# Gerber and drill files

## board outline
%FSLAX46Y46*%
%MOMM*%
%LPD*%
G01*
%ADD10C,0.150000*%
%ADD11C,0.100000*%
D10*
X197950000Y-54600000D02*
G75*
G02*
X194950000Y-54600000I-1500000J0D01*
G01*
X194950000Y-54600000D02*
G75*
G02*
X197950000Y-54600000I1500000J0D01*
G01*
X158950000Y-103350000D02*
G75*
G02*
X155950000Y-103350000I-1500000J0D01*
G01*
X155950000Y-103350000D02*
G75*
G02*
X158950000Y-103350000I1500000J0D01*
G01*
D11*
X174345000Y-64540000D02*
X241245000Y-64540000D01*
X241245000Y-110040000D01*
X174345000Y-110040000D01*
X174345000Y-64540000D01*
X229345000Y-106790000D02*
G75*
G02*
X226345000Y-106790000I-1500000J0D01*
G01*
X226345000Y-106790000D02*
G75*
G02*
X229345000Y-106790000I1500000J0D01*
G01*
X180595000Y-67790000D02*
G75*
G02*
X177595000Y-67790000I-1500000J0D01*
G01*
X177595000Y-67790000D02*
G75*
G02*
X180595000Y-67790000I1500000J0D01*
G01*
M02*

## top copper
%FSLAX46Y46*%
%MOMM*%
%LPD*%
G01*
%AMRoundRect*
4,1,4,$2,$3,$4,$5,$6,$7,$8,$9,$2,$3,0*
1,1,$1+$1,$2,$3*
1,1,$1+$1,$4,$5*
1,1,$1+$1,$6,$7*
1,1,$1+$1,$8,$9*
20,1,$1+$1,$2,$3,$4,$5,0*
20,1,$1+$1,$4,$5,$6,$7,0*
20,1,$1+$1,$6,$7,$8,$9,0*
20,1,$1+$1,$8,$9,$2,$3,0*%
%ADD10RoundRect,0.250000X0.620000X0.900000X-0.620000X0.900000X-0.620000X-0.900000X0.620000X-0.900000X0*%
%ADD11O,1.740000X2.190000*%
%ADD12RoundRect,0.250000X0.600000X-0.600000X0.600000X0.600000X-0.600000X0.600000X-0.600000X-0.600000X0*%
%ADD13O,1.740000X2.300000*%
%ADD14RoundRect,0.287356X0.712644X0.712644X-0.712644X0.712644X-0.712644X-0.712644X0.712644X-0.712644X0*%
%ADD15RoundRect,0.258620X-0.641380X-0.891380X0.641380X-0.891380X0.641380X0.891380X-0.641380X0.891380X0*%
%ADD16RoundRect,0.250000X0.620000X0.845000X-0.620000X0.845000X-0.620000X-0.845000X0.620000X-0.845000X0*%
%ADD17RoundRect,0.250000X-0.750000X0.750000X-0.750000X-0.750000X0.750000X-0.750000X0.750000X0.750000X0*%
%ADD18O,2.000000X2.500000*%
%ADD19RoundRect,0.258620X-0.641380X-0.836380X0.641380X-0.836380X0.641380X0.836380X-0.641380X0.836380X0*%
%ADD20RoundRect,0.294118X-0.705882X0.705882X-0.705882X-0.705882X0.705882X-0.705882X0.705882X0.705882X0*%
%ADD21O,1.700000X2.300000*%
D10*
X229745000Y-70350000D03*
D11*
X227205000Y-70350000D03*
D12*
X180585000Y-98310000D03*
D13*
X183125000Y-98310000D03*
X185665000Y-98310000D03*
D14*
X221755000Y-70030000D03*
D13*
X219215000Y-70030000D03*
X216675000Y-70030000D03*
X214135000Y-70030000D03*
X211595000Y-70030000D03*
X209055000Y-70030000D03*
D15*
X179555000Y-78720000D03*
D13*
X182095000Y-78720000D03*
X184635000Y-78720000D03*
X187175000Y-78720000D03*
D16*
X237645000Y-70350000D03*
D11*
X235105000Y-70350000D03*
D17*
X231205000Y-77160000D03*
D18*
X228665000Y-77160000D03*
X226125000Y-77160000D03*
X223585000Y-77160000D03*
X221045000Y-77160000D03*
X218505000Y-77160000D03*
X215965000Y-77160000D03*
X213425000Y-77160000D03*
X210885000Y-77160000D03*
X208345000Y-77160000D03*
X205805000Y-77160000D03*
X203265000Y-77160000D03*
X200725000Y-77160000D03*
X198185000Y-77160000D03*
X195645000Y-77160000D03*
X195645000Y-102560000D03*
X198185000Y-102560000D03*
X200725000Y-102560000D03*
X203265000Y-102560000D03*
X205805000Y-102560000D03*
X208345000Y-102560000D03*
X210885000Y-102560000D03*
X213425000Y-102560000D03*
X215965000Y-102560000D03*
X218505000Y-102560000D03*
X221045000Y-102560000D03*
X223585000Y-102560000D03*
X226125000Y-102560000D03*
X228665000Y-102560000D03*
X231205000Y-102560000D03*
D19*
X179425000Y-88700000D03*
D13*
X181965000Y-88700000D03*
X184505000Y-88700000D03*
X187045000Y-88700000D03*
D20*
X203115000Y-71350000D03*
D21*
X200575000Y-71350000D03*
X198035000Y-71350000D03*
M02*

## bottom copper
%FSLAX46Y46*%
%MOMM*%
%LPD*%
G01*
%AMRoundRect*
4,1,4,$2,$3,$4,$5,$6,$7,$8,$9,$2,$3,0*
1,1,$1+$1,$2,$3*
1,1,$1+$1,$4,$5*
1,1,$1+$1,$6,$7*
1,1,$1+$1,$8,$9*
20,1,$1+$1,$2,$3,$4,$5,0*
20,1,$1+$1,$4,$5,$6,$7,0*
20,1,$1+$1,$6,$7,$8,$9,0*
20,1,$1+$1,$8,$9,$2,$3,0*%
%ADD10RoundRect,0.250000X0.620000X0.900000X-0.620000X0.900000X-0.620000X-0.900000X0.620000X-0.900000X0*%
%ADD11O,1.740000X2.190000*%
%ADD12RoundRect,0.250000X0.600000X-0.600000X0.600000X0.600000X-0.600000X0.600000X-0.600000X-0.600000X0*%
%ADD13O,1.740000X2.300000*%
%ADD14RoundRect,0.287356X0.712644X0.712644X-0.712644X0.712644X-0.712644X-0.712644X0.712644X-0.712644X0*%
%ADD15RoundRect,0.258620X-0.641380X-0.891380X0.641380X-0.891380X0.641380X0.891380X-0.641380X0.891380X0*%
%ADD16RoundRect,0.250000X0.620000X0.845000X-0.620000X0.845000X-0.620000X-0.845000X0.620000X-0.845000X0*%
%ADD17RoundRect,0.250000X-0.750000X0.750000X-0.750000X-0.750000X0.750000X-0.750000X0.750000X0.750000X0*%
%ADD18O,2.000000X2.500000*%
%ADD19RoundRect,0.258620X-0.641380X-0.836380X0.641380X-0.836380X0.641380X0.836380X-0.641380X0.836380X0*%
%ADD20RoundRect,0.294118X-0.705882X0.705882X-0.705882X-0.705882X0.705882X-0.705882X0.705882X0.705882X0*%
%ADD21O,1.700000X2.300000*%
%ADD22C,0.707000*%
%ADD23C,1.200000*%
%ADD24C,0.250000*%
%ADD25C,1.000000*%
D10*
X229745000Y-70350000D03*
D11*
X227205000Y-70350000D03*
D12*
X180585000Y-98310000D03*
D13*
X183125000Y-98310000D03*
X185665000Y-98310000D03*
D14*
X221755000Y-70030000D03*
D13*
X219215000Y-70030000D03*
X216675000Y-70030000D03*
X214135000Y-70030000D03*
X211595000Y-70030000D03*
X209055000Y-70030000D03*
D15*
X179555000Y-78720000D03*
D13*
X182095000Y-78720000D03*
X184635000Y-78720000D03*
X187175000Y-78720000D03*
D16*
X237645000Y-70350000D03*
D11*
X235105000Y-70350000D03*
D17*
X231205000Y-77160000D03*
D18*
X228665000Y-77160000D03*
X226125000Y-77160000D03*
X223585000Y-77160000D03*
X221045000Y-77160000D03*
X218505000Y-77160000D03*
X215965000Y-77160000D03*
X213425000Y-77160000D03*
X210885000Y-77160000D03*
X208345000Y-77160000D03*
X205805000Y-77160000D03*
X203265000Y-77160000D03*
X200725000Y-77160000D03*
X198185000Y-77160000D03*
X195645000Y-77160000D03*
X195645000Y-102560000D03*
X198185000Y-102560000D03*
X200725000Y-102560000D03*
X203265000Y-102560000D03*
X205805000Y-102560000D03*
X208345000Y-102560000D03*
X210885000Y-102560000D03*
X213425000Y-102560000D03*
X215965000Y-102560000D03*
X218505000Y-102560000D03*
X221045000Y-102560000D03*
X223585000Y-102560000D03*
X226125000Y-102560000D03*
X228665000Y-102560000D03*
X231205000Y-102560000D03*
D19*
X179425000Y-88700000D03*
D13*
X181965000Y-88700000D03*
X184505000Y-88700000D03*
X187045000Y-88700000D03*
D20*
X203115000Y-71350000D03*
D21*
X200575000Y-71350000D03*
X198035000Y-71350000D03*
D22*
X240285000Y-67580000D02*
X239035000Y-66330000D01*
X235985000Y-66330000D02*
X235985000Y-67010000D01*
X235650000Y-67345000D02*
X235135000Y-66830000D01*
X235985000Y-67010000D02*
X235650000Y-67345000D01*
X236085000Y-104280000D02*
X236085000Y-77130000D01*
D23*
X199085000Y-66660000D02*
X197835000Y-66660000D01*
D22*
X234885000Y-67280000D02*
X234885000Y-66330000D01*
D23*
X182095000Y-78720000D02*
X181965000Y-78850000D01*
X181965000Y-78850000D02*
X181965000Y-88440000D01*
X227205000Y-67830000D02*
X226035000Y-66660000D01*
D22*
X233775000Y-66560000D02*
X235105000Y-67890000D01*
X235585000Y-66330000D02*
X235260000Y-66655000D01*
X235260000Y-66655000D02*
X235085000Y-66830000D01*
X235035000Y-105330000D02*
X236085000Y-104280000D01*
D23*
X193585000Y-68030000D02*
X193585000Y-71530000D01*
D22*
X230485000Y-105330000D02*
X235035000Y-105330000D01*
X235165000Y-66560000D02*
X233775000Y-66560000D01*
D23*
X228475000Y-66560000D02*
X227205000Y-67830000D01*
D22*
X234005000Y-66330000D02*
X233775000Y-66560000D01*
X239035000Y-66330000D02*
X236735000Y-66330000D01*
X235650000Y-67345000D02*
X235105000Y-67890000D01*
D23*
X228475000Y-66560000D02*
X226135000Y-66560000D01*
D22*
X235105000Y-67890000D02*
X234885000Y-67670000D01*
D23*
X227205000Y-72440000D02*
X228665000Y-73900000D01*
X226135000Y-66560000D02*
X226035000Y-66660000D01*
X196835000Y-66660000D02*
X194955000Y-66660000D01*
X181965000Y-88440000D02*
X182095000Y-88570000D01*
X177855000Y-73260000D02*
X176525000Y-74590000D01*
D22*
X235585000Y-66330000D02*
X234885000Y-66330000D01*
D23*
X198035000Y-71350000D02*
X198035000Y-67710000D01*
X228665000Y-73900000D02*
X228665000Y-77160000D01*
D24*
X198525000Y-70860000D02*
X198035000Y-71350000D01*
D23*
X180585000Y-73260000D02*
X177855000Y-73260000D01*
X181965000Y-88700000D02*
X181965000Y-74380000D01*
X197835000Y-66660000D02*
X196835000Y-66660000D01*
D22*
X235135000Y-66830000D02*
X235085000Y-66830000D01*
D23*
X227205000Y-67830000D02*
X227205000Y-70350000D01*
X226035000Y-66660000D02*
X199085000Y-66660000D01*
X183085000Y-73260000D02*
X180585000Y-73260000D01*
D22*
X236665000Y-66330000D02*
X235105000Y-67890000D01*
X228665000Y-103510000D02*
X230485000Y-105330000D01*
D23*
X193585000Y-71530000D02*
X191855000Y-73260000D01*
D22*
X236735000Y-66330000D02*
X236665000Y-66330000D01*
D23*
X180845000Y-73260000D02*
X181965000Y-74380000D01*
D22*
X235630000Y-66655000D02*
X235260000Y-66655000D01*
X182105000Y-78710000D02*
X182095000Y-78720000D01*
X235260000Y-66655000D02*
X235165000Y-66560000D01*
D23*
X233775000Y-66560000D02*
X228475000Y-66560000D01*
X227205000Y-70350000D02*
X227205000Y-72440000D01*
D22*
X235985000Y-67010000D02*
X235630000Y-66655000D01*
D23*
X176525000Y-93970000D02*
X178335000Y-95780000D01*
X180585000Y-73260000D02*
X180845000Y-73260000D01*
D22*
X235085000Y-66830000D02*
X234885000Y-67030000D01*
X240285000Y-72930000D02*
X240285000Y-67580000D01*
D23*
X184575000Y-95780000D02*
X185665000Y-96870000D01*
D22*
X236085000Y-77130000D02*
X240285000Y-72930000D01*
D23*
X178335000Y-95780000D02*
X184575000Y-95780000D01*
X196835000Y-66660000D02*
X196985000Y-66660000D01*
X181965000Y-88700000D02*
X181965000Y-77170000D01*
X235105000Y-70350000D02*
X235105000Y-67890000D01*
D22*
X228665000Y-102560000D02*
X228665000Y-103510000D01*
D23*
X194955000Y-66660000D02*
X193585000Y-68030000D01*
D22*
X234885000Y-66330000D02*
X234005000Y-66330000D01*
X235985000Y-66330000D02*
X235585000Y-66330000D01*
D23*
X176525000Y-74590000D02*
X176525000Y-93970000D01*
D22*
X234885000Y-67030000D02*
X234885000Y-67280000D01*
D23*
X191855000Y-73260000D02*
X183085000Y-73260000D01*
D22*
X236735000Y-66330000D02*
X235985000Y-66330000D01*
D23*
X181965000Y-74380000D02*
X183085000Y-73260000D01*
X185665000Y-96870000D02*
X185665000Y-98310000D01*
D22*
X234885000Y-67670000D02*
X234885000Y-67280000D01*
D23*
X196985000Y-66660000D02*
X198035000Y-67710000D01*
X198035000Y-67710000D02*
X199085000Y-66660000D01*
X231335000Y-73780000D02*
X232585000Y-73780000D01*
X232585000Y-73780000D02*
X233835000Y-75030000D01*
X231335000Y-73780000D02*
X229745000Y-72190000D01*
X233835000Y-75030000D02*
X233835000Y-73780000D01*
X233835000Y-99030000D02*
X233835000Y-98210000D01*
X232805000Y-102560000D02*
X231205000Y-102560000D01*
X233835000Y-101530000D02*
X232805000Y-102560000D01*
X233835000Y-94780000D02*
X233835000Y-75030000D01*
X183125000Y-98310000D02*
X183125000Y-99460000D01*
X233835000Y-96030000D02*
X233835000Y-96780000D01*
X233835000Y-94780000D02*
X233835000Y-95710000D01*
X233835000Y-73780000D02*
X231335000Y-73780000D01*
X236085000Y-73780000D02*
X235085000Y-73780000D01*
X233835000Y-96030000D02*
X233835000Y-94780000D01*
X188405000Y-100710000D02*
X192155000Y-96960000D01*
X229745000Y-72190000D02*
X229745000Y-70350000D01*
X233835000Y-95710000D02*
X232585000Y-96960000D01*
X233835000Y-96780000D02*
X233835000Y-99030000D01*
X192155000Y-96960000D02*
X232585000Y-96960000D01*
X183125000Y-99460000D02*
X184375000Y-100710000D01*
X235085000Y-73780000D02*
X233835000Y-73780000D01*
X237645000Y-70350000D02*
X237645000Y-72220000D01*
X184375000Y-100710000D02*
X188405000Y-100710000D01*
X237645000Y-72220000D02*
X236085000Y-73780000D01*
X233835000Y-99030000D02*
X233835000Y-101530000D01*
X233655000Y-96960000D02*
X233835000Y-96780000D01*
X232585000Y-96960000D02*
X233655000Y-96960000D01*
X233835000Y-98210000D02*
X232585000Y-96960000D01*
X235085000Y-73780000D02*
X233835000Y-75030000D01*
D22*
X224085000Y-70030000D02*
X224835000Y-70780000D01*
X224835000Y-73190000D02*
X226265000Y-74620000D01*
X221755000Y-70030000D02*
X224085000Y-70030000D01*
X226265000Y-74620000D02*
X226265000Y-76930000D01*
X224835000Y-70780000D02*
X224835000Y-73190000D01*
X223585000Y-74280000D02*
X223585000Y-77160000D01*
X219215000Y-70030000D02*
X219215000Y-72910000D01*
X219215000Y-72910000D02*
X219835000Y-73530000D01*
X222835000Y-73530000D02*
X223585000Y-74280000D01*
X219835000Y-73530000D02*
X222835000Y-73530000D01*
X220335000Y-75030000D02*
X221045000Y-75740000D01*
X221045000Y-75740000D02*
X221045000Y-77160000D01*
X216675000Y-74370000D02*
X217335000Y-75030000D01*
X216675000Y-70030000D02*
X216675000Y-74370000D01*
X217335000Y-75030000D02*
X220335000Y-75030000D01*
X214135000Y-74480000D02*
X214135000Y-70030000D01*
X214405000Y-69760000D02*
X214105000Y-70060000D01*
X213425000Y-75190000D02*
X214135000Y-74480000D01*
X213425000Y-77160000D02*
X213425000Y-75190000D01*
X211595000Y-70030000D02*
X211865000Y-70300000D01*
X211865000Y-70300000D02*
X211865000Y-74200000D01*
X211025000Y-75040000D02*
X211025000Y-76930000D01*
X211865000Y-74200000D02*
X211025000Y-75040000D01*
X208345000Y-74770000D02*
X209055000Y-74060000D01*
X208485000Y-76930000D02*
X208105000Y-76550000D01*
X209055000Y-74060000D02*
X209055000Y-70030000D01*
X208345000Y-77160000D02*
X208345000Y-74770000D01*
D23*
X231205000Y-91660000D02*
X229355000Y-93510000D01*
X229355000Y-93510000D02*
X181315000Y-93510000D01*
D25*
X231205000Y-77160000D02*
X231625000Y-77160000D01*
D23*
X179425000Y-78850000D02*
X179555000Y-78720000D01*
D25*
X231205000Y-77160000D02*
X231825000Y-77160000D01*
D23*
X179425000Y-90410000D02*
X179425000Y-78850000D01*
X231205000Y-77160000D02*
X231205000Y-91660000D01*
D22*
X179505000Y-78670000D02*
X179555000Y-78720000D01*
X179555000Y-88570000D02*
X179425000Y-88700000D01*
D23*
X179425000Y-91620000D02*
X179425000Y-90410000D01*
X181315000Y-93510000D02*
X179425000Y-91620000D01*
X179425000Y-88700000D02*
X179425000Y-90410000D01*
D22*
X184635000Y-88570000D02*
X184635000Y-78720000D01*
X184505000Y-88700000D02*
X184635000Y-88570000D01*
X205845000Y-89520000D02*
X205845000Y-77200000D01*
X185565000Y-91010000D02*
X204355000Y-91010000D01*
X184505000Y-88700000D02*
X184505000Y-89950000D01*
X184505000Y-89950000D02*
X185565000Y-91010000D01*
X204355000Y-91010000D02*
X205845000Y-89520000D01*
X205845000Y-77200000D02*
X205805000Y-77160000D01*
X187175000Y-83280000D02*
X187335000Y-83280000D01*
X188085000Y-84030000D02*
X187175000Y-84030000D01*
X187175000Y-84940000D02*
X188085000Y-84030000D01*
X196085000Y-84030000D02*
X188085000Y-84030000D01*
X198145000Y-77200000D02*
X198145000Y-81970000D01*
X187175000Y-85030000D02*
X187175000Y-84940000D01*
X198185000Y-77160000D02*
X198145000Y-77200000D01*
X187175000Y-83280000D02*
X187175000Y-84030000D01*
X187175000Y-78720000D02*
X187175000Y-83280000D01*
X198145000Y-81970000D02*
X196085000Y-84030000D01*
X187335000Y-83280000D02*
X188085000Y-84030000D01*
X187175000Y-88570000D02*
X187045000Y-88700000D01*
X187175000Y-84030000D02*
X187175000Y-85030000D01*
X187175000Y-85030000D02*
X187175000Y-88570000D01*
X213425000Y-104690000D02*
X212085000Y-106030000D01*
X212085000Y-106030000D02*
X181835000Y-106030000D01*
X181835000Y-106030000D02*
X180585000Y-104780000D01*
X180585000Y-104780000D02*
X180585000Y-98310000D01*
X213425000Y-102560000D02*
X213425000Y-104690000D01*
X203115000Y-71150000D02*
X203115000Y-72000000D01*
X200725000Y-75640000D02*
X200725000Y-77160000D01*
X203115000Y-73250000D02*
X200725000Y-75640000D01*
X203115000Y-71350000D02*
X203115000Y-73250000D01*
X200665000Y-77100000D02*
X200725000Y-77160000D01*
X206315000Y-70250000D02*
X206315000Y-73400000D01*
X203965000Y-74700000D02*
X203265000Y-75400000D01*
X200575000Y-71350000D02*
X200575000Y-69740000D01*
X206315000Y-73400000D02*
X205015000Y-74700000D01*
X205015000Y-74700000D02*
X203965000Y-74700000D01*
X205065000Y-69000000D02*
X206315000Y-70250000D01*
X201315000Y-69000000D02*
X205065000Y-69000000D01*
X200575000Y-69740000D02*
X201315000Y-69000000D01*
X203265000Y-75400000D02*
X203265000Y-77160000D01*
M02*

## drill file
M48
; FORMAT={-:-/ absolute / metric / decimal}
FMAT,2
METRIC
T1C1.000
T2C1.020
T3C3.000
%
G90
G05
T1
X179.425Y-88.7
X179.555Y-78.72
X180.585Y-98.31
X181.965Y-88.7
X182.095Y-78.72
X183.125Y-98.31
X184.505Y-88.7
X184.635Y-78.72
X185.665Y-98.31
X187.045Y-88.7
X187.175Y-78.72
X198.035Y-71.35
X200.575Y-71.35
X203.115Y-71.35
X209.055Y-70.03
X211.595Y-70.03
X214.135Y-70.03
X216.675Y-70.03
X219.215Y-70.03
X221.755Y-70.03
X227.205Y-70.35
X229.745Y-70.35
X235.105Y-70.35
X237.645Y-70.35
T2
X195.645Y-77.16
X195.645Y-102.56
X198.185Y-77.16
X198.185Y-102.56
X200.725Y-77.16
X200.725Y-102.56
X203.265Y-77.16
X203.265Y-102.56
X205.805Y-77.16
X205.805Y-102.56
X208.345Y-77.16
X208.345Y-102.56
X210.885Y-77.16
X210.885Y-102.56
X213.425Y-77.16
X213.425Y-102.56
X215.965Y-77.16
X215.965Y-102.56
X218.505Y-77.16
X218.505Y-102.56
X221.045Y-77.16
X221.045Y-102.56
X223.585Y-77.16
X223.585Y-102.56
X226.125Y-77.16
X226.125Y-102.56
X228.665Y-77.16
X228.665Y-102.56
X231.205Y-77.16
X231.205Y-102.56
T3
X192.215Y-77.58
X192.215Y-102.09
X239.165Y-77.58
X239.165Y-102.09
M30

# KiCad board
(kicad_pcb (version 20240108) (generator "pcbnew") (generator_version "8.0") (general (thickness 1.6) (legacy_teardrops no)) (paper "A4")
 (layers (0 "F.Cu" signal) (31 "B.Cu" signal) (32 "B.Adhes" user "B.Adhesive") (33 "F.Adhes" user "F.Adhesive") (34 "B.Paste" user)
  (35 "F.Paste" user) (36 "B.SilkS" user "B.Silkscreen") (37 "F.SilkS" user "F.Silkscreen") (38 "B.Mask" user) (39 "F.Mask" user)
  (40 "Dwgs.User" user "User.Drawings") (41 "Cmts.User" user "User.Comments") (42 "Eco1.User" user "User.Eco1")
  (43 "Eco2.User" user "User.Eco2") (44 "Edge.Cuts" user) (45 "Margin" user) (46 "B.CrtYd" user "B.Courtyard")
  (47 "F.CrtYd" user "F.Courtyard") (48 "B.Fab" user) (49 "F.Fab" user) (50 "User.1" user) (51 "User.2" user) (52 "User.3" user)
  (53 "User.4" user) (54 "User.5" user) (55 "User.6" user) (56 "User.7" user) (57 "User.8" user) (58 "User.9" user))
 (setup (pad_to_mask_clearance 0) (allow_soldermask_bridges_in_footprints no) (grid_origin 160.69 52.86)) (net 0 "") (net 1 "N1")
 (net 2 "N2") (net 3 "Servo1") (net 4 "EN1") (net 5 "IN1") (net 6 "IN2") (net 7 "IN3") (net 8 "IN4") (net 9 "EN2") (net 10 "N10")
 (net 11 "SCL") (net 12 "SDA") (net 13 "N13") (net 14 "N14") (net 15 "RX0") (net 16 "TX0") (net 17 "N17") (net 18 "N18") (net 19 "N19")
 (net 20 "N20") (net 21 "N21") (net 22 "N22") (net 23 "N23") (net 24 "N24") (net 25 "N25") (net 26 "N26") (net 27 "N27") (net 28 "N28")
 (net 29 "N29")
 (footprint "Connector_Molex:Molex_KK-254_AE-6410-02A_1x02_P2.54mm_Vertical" (layer "F.Cu") (at 229.745 70.35 180)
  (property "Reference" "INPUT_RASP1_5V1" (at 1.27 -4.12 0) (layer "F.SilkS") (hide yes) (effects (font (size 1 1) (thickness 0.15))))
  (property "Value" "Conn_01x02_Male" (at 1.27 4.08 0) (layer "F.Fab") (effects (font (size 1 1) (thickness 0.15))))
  (pad "1" thru_hole roundrect (at 0 0 180) (size 1.74 2.3) (drill 1) (layers "*.Cu" "*.Mask") (remove_unused_layers no)
   (roundrect_rratio 0.143678) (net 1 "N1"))
  (pad "2" thru_hole oval (at 2.54 0 180) (size 1.74 2.19) (drill 1) (layers "*.Cu" "*.Mask") (remove_unused_layers no) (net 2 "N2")))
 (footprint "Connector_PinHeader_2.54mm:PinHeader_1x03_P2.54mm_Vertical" (layer "F.Cu") (at 180.585 98.31 90)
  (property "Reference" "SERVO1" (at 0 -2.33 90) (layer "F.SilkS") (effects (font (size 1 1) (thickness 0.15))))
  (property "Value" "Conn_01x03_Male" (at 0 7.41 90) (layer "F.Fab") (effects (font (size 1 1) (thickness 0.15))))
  (pad "1" thru_hole roundrect (at 0 0 90) (size 1.7 1.7) (drill 1) (layers "*.Cu" "*.Mask") (remove_unused_layers no)
   (roundrect_rratio 0.1470588235) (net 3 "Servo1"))
  (pad "2" thru_hole oval (at 0 2.54 90) (size 2.3 1.74) (drill 1) (layers "*.Cu" "*.Mask") (remove_unused_layers no) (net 1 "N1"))
  (pad "3" thru_hole oval (at 0 5.08 90) (size 2.3 1.74) (drill 1) (layers "*.Cu" "*.Mask") (remove_unused_layers no) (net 2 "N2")))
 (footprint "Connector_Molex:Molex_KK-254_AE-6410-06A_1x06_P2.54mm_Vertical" (layer "F.Cu") (at 221.755 70.03 180)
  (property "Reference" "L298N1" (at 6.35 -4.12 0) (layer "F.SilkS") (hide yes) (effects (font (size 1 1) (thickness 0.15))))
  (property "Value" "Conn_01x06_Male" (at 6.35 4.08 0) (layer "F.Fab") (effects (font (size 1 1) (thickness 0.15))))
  (pad "1" thru_hole roundrect (at 0 0 180) (size 2 2) (drill 1) (layers "*.Cu" "*.Mask") (remove_unused_layers no)
   (roundrect_rratio 0.143678) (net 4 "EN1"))
  (pad "2" thru_hole oval (at 2.54 0 180) (size 1.74 2.3) (drill 1) (layers "*.Cu" "*.Mask") (remove_unused_layers no) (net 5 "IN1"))
  (pad "3" thru_hole oval (at 5.08 0 180) (size 1.74 2.3) (drill 1) (layers "*.Cu" "*.Mask") (remove_unused_layers no) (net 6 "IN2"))
  (pad "4" thru_hole oval (at 7.62 0 180) (size 1.74 2.3) (drill 1) (layers "*.Cu" "*.Mask") (remove_unused_layers no) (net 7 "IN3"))
  (pad "5" thru_hole oval (at 10.16 0 180) (size 1.74 2.3) (drill 1) (layers "*.Cu" "*.Mask") (remove_unused_layers no) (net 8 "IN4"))
  (pad "6" thru_hole oval (at 12.7 0 180) (size 1.74 2.3) (drill 1) (layers "*.Cu" "*.Mask") (remove_unused_layers no) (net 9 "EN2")))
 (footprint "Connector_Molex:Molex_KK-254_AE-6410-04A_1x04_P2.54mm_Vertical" (layer "F.Cu") (at 179.555 78.72)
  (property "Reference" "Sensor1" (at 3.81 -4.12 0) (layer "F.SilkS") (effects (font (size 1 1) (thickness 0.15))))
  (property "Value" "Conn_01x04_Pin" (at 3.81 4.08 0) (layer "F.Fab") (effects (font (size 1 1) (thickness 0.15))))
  (pad "1" thru_hole roundrect (at 0 0) (size 1.8 2.3) (drill 1) (layers "*.Cu" "*.Mask") (remove_unused_layers no)
   (roundrect_rratio 0.143678) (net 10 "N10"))
  (pad "2" thru_hole oval (at 2.54 0) (size 1.74 2.3) (drill 1) (layers "*.Cu" "*.Mask") (remove_unused_layers no) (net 2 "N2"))
  (pad "3" thru_hole oval (at 5.08 0) (size 1.74 2.3) (drill 1) (layers "*.Cu" "*.Mask") (remove_unused_layers no) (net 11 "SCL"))
  (pad "4" thru_hole oval (at 7.62 0) (size 1.74 2.3) (drill 1) (layers "*.Cu" "*.Mask") (remove_unused_layers no) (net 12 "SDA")))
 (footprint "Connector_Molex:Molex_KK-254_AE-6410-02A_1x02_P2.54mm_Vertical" (layer "F.Cu") (at 237.645 70.35 180)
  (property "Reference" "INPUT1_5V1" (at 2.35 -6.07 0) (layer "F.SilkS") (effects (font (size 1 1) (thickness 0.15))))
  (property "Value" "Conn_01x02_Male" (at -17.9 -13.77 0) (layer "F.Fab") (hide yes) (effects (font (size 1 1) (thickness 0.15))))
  (pad "1" thru_hole roundrect (at 0 0 180) (size 1.74 2.19) (drill 1) (layers "*.Cu" "*.Mask") (remove_unused_layers no)
   (roundrect_rratio 0.143678) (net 1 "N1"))
  (pad "2" thru_hole oval (at 2.54 0 180) (size 1.74 2.19) (drill 1) (layers "*.Cu" "*.Mask") (remove_unused_layers no) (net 2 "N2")))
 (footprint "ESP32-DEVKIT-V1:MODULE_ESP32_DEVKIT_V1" (layer "F.Cu") (at 215.69 89.86 -90)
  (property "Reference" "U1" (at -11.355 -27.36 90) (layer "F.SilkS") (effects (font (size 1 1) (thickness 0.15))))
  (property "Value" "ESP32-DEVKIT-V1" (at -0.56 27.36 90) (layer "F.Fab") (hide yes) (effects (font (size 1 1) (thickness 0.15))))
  (pad "" np_thru_hole circle (at -12.28 -23.475 270) (size 3 3) (drill 3) (layers "*.Cu" "*.Mask"))
  (pad "" np_thru_hole circle (at -12.28 23.475 270) (size 3 3) (drill 3) (layers "*.Cu" "*.Mask"))
  (pad "" np_thru_hole circle (at 12.23 -23.475 270) (size 3 3) (drill 3) (layers "*.Cu" "*.Mask"))
  (pad "" np_thru_hole circle (at 12.23 23.475 270) (size 3 3) (drill 3) (layers "*.Cu" "*.Mask"))
  (pad "1" thru_hole roundrect (at -12.7 -15.515 270) (size 2 2) (drill 1.02) (layers "*.Cu" "*.Mask") (remove_unused_layers no)
   (roundrect_rratio 0.125) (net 10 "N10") (solder_mask_margin 0.102))
  (pad "2" thru_hole oval (at -12.7 -12.975 270) (size 2.5 2) (drill 1.02) (layers "*.Cu" "*.Mask") (remove_unused_layers no) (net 2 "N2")
   (solder_mask_margin 0.102))
  (pad "3" thru_hole oval (at -12.7 -10.435 270) (size 2.5 2) (drill 1.02) (layers "*.Cu" "*.Mask") (remove_unused_layers no) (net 4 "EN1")
   (solder_mask_margin 0.102))
  (pad "4" thru_hole oval (at -12.7 -7.895 270) (size 2.5 2) (drill 1.02) (layers "*.Cu" "*.Mask") (remove_unused_layers no) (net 5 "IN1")
   (solder_mask_margin 0.102))
  (pad "5" thru_hole oval (at -12.7 -5.355 270) (size 2.5 2) (drill 1.02) (layers "*.Cu" "*.Mask") (remove_unused_layers no) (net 6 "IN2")
   (solder_mask_margin 0.102))
  (pad "6" thru_hole oval (at -12.7 -2.815 270) (size 2.5 2) (drill 1.02) (layers "*.Cu" "*.Mask") (remove_unused_layers no) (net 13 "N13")
   (solder_mask_margin 0.102))
  (pad "7" thru_hole oval (at -12.7 -0.275 270) (size 2.5 2) (drill 1.02) (layers "*.Cu" "*.Mask") (remove_unused_layers no) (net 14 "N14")
   (solder_mask_margin 0.102))
  (pad "8" thru_hole oval (at -12.7 2.265 270) (size 2.5 2) (drill 1.02) (layers "*.Cu" "*.Mask") (remove_unused_layers no) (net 7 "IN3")
   (solder_mask_margin 0.102))
  (pad "9" thru_hole oval (at -12.7 4.805 270) (size 2.5 2) (drill 1.02) (layers "*.Cu" "*.Mask") (remove_unused_layers no) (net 8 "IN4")
   (solder_mask_margin 0.102))
  (pad "10" thru_hole oval (at -12.7 7.345 270) (size 2.5 2) (drill 1.02) (layers "*.Cu" "*.Mask") (remove_unused_layers no) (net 9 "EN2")
   (solder_mask_margin 0.102))
  (pad "11" thru_hole oval (at -12.7 9.885 270) (size 2.5 2) (drill 1.02) (layers "*.Cu" "*.Mask") (remove_unused_layers no) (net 11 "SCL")
   (solder_mask_margin 0.102))
  (pad "12" thru_hole oval (at -12.7 12.425 270) (size 2.5 2) (drill 1.02) (layers "*.Cu" "*.Mask") (remove_unused_layers no) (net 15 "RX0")
   (solder_mask_margin 0.102))
  (pad "13" thru_hole oval (at -12.7 14.965 270) (size 2.5 2) (drill 1.02) (layers "*.Cu" "*.Mask") (remove_unused_layers no) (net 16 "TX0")
   (solder_mask_margin 0.102))
  (pad "14" thru_hole oval (at -12.7 17.505 270) (size 2.5 2) (drill 1.02) (layers "*.Cu" "*.Mask") (remove_unused_layers no) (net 12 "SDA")
   (solder_mask_margin 0.102))
  (pad "15" thru_hole oval (at -12.7 20.045 270) (size 2.5 2) (drill 1.02) (layers "*.Cu" "*.Mask") (remove_unused_layers no) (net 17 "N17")
   (solder_mask_margin 0.102))
  (pad "16" thru_hole oval (at 12.7 20.045 270) (size 2.5 2) (drill 1.02) (layers "*.Cu" "*.Mask") (remove_unused_layers no) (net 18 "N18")
   (solder_mask_margin 0.102))
  (pad "17" thru_hole oval (at 12.7 17.505 270) (size 2.5 2) (drill 1.02) (layers "*.Cu" "*.Mask") (remove_unused_layers no) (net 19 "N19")
   (solder_mask_margin 0.102))
  (pad "18" thru_hole oval (at 12.7 14.965 270) (size 2.5 2) (drill 1.02) (layers "*.Cu" "*.Mask") (remove_unused_layers no) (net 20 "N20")
   (solder_mask_margin 0.102))
  (pad "19" thru_hole oval (at 12.7 12.425 270) (size 2.5 2) (drill 1.02) (layers "*.Cu" "*.Mask") (remove_unused_layers no) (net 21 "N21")
   (solder_mask_margin 0.102))
  (pad "20" thru_hole oval (at 12.7 9.885 270) (size 2.5 2) (drill 1.02) (layers "*.Cu" "*.Mask") (remove_unused_layers no) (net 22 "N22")
   (solder_mask_margin 0.102))
  (pad "21" thru_hole oval (at 12.7 7.345 270) (size 2.5 2) (drill 1.02) (layers "*.Cu" "*.Mask") (remove_unused_layers no) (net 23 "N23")
   (solder_mask_margin 0.102))
  (pad "22" thru_hole oval (at 12.7 4.805 270) (size 2.5 2) (drill 1.02) (layers "*.Cu" "*.Mask") (remove_unused_layers no) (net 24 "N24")
   (solder_mask_margin 0.102))
  (pad "23" thru_hole oval (at 12.7 2.265 270) (size 2.5 2) (drill 1.02) (layers "*.Cu" "*.Mask") (remove_unused_layers no) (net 3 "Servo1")
   (solder_mask_margin 0.102))
  (pad "24" thru_hole oval (at 12.7 -0.275 270) (size 2.5 2) (drill 1.02) (layers "*.Cu" "*.Mask") (remove_unused_layers no) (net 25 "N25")
   (solder_mask_margin 0.102))
  (pad "25" thru_hole oval (at 12.7 -2.815 270) (size 2.5 2) (drill 1.02) (layers "*.Cu" "*.Mask") (remove_unused_layers no) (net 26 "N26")
   (solder_mask_margin 0.102))
  (pad "26" thru_hole oval (at 12.7 -5.355 270) (size 2.5 2) (drill 1.02) (layers "*.Cu" "*.Mask") (remove_unused_layers no) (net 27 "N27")
   (solder_mask_margin 0.102))
  (pad "27" thru_hole oval (at 12.7 -7.895 270) (size 2.5 2) (drill 1.02) (layers "*.Cu" "*.Mask") (remove_unused_layers no) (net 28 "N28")
   (solder_mask_margin 0.102))
  (pad "28" thru_hole oval (at 12.7 -10.435 270) (size 2.5 2) (drill 1.02) (layers "*.Cu" "*.Mask") (remove_unused_layers no) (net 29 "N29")
   (solder_mask_margin 0.102))
  (pad "29" thru_hole oval (at 12.7 -12.975 270) (size 2.5 2) (drill 1.02) (layers "*.Cu" "*.Mask") (remove_unused_layers no) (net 2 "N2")
   (solder_mask_margin 0.102))
  (pad "30" thru_hole oval (at 12.7 -15.515 270) (size 2.5 2) (drill 1.02) (layers "*.Cu" "*.Mask") (remove_unused_layers no) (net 1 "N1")
   (solder_mask_margin 0.102)))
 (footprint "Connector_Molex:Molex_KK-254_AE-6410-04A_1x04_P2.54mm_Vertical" (layer "F.Cu") (at 179.425 88.7)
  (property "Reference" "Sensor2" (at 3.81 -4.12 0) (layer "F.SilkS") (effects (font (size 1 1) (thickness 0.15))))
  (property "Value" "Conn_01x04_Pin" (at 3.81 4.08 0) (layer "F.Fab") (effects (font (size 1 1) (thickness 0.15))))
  (pad "1" thru_hole roundrect (at 0 0) (size 1.8 2.19) (drill 1) (layers "*.Cu" "*.Mask") (remove_unused_layers no)
   (roundrect_rratio 0.143678) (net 10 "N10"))
  (pad "2" thru_hole oval (at 2.54 0) (size 1.74 2.3) (drill 1) (layers "*.Cu" "*.Mask") (remove_unused_layers no) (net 2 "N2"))
  (pad "3" thru_hole oval (at 5.08 0) (size 1.74 2.3) (drill 1) (layers "*.Cu" "*.Mask") (remove_unused_layers no) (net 11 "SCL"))
  (pad "4" thru_hole oval (at 7.62 0) (size 1.74 2.3) (drill 1) (layers "*.Cu" "*.Mask") (remove_unused_layers no) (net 12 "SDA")))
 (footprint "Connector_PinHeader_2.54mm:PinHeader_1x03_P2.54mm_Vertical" (layer "F.Cu") (at 203.115 71.35 -90)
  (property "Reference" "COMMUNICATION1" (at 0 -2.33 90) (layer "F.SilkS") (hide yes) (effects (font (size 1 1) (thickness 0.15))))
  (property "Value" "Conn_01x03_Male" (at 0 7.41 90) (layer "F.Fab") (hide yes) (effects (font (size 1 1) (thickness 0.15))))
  (pad "1" thru_hole roundrect (at 0 0 270) (size 2 2) (drill 1) (layers "*.Cu" "*.Mask") (remove_unused_layers no)
   (roundrect_rratio 0.1470588235) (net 16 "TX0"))
  (pad "2" thru_hole oval (at 0 2.54 270) (size 2.3 1.7) (drill 1) (layers "*.Cu" "*.Mask") (remove_unused_layers no) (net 15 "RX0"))
  (pad "3" thru_hole oval (at 0 5.08 270) (size 2.3 1.7) (drill 1) (layers "*.Cu" "*.Mask") (remove_unused_layers no) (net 2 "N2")))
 (gr_circle (center 196.45 54.6) (end 197.95 54.6) (locked yes) (stroke (width 0.15) (type solid)) (fill none) (layer "Edge.Cuts"))
 (gr_circle (center 157.45 103.35) (end 158.95 103.35) (locked yes) (stroke (width 0.15) (type solid)) (fill none) (layer "Edge.Cuts"))
 (gr_rect (start 174.345 64.54) (end 241.245 110.04) (stroke (width 0.1) (type default)) (fill none) (layer "Edge.Cuts"))
 (gr_circle (center 227.845 106.79) (end 227.845 108.29) (stroke (width 0.1) (type default)) (fill none) (layer "Edge.Cuts"))
 (gr_circle (center 179.095 67.79) (end 179.095 69.29) (stroke (width 0.1) (type default)) (fill none) (layer "Edge.Cuts"))
 (segment (start 240.285 67.58) (end 239.035 66.33) (width 0.707) (layer "B.Cu") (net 2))
 (segment (start 235.985 66.33) (end 235.985 67.01) (width 0.707) (layer "B.Cu") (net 2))
 (segment (start 235.65 67.345) (end 235.135 66.83) (width 0.707) (layer "B.Cu") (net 2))
 (segment (start 235.985 67.01) (end 235.65 67.345) (width 0.707) (layer "B.Cu") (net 2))
 (segment (start 236.085 104.28) (end 236.085 77.13) (width 0.707) (layer "B.Cu") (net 2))
 (segment (start 199.085 66.66) (end 197.835 66.66) (width 1.2) (layer "B.Cu") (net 2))
 (segment (start 234.885 67.28) (end 234.885 66.33) (width 0.707) (layer "B.Cu") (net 2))
 (segment (start 182.095 78.72) (end 181.965 78.85) (width 1.2) (layer "B.Cu") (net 2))
 (segment (start 181.965 78.85) (end 181.965 88.44) (width 1.2) (layer "B.Cu") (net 2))
 (segment (start 227.205 67.83) (end 226.035 66.66) (width 1.2) (layer "B.Cu") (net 2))
 (segment (start 233.775 66.56) (end 235.105 67.89) (width 0.707) (layer "B.Cu") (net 2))
 (segment (start 235.585 66.33) (end 235.26 66.655) (width 0.707) (layer "B.Cu") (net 2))
 (segment (start 235.26 66.655) (end 235.085 66.83) (width 0.707) (layer "B.Cu") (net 2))
 (segment (start 235.035 105.33) (end 236.085 104.28) (width 0.707) (layer "B.Cu") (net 2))
 (segment (start 193.585 68.03) (end 193.585 71.53) (width 1.2) (layer "B.Cu") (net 2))
 (segment (start 230.485 105.33) (end 235.035 105.33) (width 0.707) (layer "B.Cu") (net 2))
 (segment (start 235.165 66.56) (end 233.775 66.56) (width 0.707) (layer "B.Cu") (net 2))
 (segment (start 228.475 66.56) (end 227.205 67.83) (width 1.2) (layer "B.Cu") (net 2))
 (segment (start 234.005 66.33) (end 233.775 66.56) (width 0.707) (layer "B.Cu") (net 2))
 (segment (start 239.035 66.33) (end 236.735 66.33) (width 0.707) (layer "B.Cu") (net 2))
 (segment (start 235.65 67.345) (end 235.105 67.89) (width 0.707) (layer "B.Cu") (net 2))
 (segment (start 228.475 66.56) (end 226.135 66.56) (width 1.2) (layer "B.Cu") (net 2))
 (segment (start 235.105 67.89) (end 234.885 67.67) (width 0.707) (layer "B.Cu") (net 2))
 (segment (start 227.205 72.44) (end 228.665 73.9) (width 1.2) (layer "B.Cu") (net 2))
 (segment (start 226.135 66.56) (end 226.035 66.66) (width 1.2) (layer "B.Cu") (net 2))
 (segment (start 196.835 66.66) (end 194.955 66.66) (width 1.2) (layer "B.Cu") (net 2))
 (segment (start 181.965 88.44) (end 182.095 88.57) (width 1.2) (layer "B.Cu") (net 2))
 (segment (start 177.855 73.26) (end 176.525 74.59) (width 1.2) (layer "B.Cu") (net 2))
 (segment (start 235.585 66.33) (end 234.885 66.33) (width 0.707) (layer "B.Cu") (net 2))
 (segment (start 198.035 71.35) (end 198.035 67.71) (width 1.2) (layer "B.Cu") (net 2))
 (segment (start 228.665 73.9) (end 228.665 77.16) (width 1.2) (layer "B.Cu") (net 2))
 (segment (start 198.525 70.86) (end 198.035 71.35) (width 0.25) (layer "B.Cu") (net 2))
 (segment (start 180.585 73.26) (end 177.855 73.26) (width 1.2) (layer "B.Cu") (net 2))
 (segment (start 181.965 88.7) (end 181.965 74.38) (width 1.2) (layer "B.Cu") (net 2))
 (segment (start 197.835 66.66) (end 196.835 66.66) (width 1.2) (layer "B.Cu") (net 2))
 (segment (start 235.135 66.83) (end 235.085 66.83) (width 0.707) (layer "B.Cu") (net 2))
 (segment (start 227.205 67.83) (end 227.205 70.35) (width 1.2) (layer "B.Cu") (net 2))
 (segment (start 226.035 66.66) (end 199.085 66.66) (width 1.2) (layer "B.Cu") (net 2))
 (segment (start 183.085 73.26) (end 180.585 73.26) (width 1.2) (layer "B.Cu") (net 2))
 (segment (start 236.665 66.33) (end 235.105 67.89) (width 0.707) (layer "B.Cu") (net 2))
 (segment (start 228.665 103.51) (end 230.485 105.33) (width 0.707) (layer "B.Cu") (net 2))
 (segment (start 193.585 71.53) (end 191.855 73.26) (width 1.2) (layer "B.Cu") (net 2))
 (segment (start 236.735 66.33) (end 236.665 66.33) (width 0.707) (layer "B.Cu") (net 2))
 (segment (start 180.845 73.26) (end 181.965 74.38) (width 1.2) (layer "B.Cu") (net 2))
 (segment (start 235.63 66.655) (end 235.26 66.655) (width 0.707) (layer "B.Cu") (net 2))
 (segment (start 182.105 78.71) (end 182.095 78.72) (width 0.707) (layer "B.Cu") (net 2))
 (segment (start 235.26 66.655) (end 235.165 66.56) (width 0.707) (layer "B.Cu") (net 2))
 (segment (start 233.775 66.56) (end 228.475 66.56) (width 1.2) (layer "B.Cu") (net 2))
 (segment (start 227.205 70.35) (end 227.205 72.44) (width 1.2) (layer "B.Cu") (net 2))
 (segment (start 235.985 67.01) (end 235.63 66.655) (width 0.707) (layer "B.Cu") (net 2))
 (segment (start 176.525 93.97) (end 178.335 95.78) (width 1.2) (layer "B.Cu") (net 2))
 (segment (start 180.585 73.26) (end 180.845 73.26) (width 1.2) (layer "B.Cu") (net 2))
 (segment (start 235.085 66.83) (end 234.885 67.03) (width 0.707) (layer "B.Cu") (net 2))
 (segment (start 240.285 72.93) (end 240.285 67.58) (width 0.707) (layer "B.Cu") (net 2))
 (segment (start 184.575 95.78) (end 185.665 96.87) (width 1.2) (layer "B.Cu") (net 2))
 (segment (start 236.085 77.13) (end 240.285 72.93) (width 0.707) (layer "B.Cu") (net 2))
 (segment (start 178.335 95.78) (end 184.575 95.78) (width 1.2) (layer "B.Cu") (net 2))
 (segment (start 196.835 66.66) (end 196.985 66.66) (width 1.2) (layer "B.Cu") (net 2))
 (segment (start 181.965 88.7) (end 181.965 77.17) (width 1.2) (layer "B.Cu") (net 2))
 (segment (start 235.105 70.35) (end 235.105 67.89) (width 1.2) (layer "B.Cu") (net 2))
 (segment (start 228.665 102.56) (end 228.665 103.51) (width 0.707) (layer "B.Cu") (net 2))
 (segment (start 194.955 66.66) (end 193.585 68.03) (width 1.2) (layer "B.Cu") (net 2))
 (segment (start 234.885 66.33) (end 234.005 66.33) (width 0.707) (layer "B.Cu") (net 2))
 (segment (start 235.985 66.33) (end 235.585 66.33) (width 0.707) (layer "B.Cu") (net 2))
 (segment (start 176.525 74.59) (end 176.525 93.97) (width 1.2) (layer "B.Cu") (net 2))
 (segment (start 234.885 67.03) (end 234.885 67.28) (width 0.707) (layer "B.Cu") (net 2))
 (segment (start 191.855 73.26) (end 183.085 73.26) (width 1.2) (layer "B.Cu") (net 2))
 (segment (start 236.735 66.33) (end 235.985 66.33) (width 0.707) (layer "B.Cu") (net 2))
 (segment (start 181.965 74.38) (end 183.085 73.26) (width 1.2) (layer "B.Cu") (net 2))
 (segment (start 185.665 96.87) (end 185.665 98.31) (width 1.2) (layer "B.Cu") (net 2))
 (segment (start 234.885 67.67) (end 234.885 67.28) (width 0.707) (layer "B.Cu") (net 2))
 (segment (start 196.985 66.66) (end 198.035 67.71) (width 1.2) (layer "B.Cu") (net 2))
 (segment (start 198.035 67.71) (end 199.085 66.66) (width 1.2) (layer "B.Cu") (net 2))
 (segment (start 231.335 73.78) (end 232.585 73.78) (width 1.2) (layer "B.Cu") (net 1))
 (segment (start 232.585 73.78) (end 233.835 75.03) (width 1.2) (layer "B.Cu") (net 1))
 (segment (start 231.335 73.78) (end 229.745 72.19) (width 1.2) (layer "B.Cu") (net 1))
 (segment (start 233.835 75.03) (end 233.835 73.78) (width 1.2) (layer "B.Cu") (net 1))
 (segment (start 233.835 99.03) (end 233.835 98.21) (width 1.2) (layer "B.Cu") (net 1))
 (segment (start 232.805 102.56) (end 231.205 102.56) (width 1.2) (layer "B.Cu") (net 1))
 (segment (start 233.835 101.53) (end 232.805 102.56) (width 1.2) (layer "B.Cu") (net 1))
 (segment (start 233.835 94.78) (end 233.835 75.03) (width 1.2) (layer "B.Cu") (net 1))
 (segment (start 183.125 98.31) (end 183.125 99.46) (width 1.2) (layer "B.Cu") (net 1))
 (segment (start 233.835 96.03) (end 233.835 96.78) (width 1.2) (layer "B.Cu") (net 1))
 (segment (start 233.835 94.78) (end 233.835 95.71) (width 1.2) (layer "B.Cu") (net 1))
 (segment (start 233.835 73.78) (end 231.335 73.78) (width 1.2) (layer "B.Cu") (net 1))
 (segment (start 236.085 73.78) (end 235.085 73.78) (width 1.2) (layer "B.Cu") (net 1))
 (segment (start 233.835 96.03) (end 233.835 94.78) (width 1.2) (layer "B.Cu") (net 1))
 (segment (start 188.405 100.71) (end 192.155 96.96) (width 1.2) (layer "B.Cu") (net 1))
 (segment (start 229.745 72.19) (end 229.745 70.35) (width 1.2) (layer "B.Cu") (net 1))
 (segment (start 233.835 95.71) (end 232.585 96.96) (width 1.2) (layer "B.Cu") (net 1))
 (segment (start 233.835 96.78) (end 233.835 99.03) (width 1.2) (layer "B.Cu") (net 1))
 (segment (start 192.155 96.96) (end 232.585 96.96) (width 1.2) (layer "B.Cu") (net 1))
 (segment (start 183.125 99.46) (end 184.375 100.71) (width 1.2) (layer "B.Cu") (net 1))
 (segment (start 235.085 73.78) (end 233.835 73.78) (width 1.2) (layer "B.Cu") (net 1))
 (segment (start 237.645 70.35) (end 237.645 72.22) (width 1.2) (layer "B.Cu") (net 1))
 (segment (start 184.375 100.71) (end 188.405 100.71) (width 1.2) (layer "B.Cu") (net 1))
 (segment (start 237.645 72.22) (end 236.085 73.78) (width 1.2) (layer "B.Cu") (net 1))
 (segment (start 233.835 99.03) (end 233.835 101.53) (width 1.2) (layer "B.Cu") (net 1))
 (segment (start 233.655 96.96) (end 233.835 96.78) (width 1.2) (layer "B.Cu") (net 1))
 (segment (start 232.585 96.96) (end 233.655 96.96) (width 1.2) (layer "B.Cu") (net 1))
 (segment (start 233.835 98.21) (end 232.585 96.96) (width 1.2) (layer "B.Cu") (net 1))
 (segment (start 235.085 73.78) (end 233.835 75.03) (width 1.2) (layer "B.Cu") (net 1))
 (segment (start 224.085 70.03) (end 224.835 70.78) (width 0.707) (layer "B.Cu") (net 4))
 (segment (start 224.835 73.19) (end 226.265 74.62) (width 0.707) (layer "B.Cu") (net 4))
 (segment (start 221.755 70.03) (end 224.085 70.03) (width 0.707) (layer "B.Cu") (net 4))
 (segment (start 226.265 74.62) (end 226.265 76.93) (width 0.707) (layer "B.Cu") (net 4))
 (segment (start 224.835 70.78) (end 224.835 73.19) (width 0.707) (layer "B.Cu") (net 4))
 (segment (start 223.585 74.28) (end 223.585 77.16) (width 0.707) (layer "B.Cu") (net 5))
 (segment (start 219.215 70.03) (end 219.215 72.91) (width 0.707) (layer "B.Cu") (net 5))
 (segment (start 219.215 72.91) (end 219.835 73.53) (width 0.707) (layer "B.Cu") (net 5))
 (segment (start 222.835 73.53) (end 223.585 74.28) (width 0.707) (layer "B.Cu") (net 5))
 (segment (start 219.835 73.53) (end 222.835 73.53) (width 0.707) (layer "B.Cu") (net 5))
 (segment (start 220.335 75.03) (end 221.045 75.74) (width 0.707) (layer "B.Cu") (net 6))
 (segment (start 221.045 75.74) (end 221.045 77.16) (width 0.707) (layer "B.Cu") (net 6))
 (segment (start 216.675 74.37) (end 217.335 75.03) (width 0.707) (layer "B.Cu") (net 6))
 (segment (start 216.675 70.03) (end 216.675 74.37) (width 0.707) (layer "B.Cu") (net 6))
 (segment (start 217.335 75.03) (end 220.335 75.03) (width 0.707) (layer "B.Cu") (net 6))
 (segment (start 214.135 74.48) (end 214.135 70.03) (width 0.707) (layer "B.Cu") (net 7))
 (segment (start 214.405 69.76) (end 214.105 70.06) (width 0.707) (layer "B.Cu") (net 7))
 (segment (start 213.425 75.19) (end 214.135 74.48) (width 0.707) (layer "B.Cu") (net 7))
 (segment (start 213.425 77.16) (end 213.425 75.19) (width 0.707) (layer "B.Cu") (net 7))
 (segment (start 211.595 70.03) (end 211.865 70.3) (width 0.707) (layer "B.Cu") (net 8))
 (segment (start 211.865 70.3) (end 211.865 74.2) (width 0.707) (layer "B.Cu") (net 8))
 (segment (start 211.025 75.04) (end 211.025 76.93) (width 0.707) (layer "B.Cu") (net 8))
 (segment (start 211.865 74.2) (end 211.025 75.04) (width 0.707) (layer "B.Cu") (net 8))
 (segment (start 208.345 74.77) (end 209.055 74.06) (width 0.707) (layer "B.Cu") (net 9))
 (segment (start 208.485 76.93) (end 208.105 76.55) (width 0.707) (layer "B.Cu") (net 9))
 (segment (start 209.055 74.06) (end 209.055 70.03) (width 0.707) (layer "B.Cu") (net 9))
 (segment (start 208.345 77.16) (end 208.345 74.77) (width 0.707) (layer "B.Cu") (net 9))
 (segment (start 231.205 91.66) (end 229.355 93.51) (width 1.2) (layer "B.Cu") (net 10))
 (segment (start 229.355 93.51) (end 181.315 93.51) (width 1.2) (layer "B.Cu") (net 10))
 (segment (start 231.205 77.16) (end 231.625 77.16) (width 1) (layer "B.Cu") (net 10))
 (segment (start 179.425 78.85) (end 179.555 78.72) (width 1.2) (layer "B.Cu") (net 10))
 (segment (start 231.205 77.16) (end 231.825 77.16) (width 1) (layer "B.Cu") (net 10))
 (segment (start 179.425 90.41) (end 179.425 78.85) (width 1.2) (layer "B.Cu") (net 10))
 (segment (start 231.205 77.16) (end 231.205 91.66) (width 1.2) (layer "B.Cu") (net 10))
 (segment (start 179.505 78.67) (end 179.555 78.72) (width 0.707) (layer "B.Cu") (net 10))
 (segment (start 179.555 88.57) (end 179.425 88.7) (width 0.707) (layer "B.Cu") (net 10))
 (segment (start 179.425 91.62) (end 179.425 90.41) (width 1.2) (layer "B.Cu") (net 10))
 (segment (start 181.315 93.51) (end 179.425 91.62) (width 1.2) (layer "B.Cu") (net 10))
 (segment (start 179.425 88.7) (end 179.425 90.41) (width 1.2) (layer "B.Cu") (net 10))
 (segment (start 184.635 88.57) (end 184.635 78.72) (width 0.707) (layer "B.Cu") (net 11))
 (segment (start 184.505 88.7) (end 184.635 88.57) (width 0.707) (layer "B.Cu") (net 11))
 (segment (start 205.845 89.52) (end 205.845 77.2) (width 0.707) (layer "B.Cu") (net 11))
 (segment (start 185.565 91.01) (end 204.355 91.01) (width 0.707) (layer "B.Cu") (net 11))
 (segment (start 184.505 88.7) (end 184.505 89.95) (width 0.707) (layer "B.Cu") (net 11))
 (segment (start 184.505 89.95) (end 185.565 91.01) (width 0.707) (layer "B.Cu") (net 11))
 (segment (start 204.355 91.01) (end 205.845 89.52) (width 0.707) (layer "B.Cu") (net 11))
 (segment (start 205.845 77.2) (end 205.805 77.16) (width 0.707) (layer "B.Cu") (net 11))
 (segment (start 187.175 83.28) (end 187.335 83.28) (width 0.707) (layer "B.Cu") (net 12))
 (segment (start 188.085 84.03) (end 187.175 84.03) (width 0.707) (layer "B.Cu") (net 12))
 (segment (start 187.175 84.94) (end 188.085 84.03) (width 0.707) (layer "B.Cu") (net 12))
 (segment (start 196.085 84.03) (end 188.085 84.03) (width 0.707) (layer "B.Cu") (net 12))
 (segment (start 198.145 77.2) (end 198.145 81.97) (width 0.707) (layer "B.Cu") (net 12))
 (segment (start 187.175 85.03) (end 187.175 84.94) (width 0.707) (layer "B.Cu") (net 12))
 (segment (start 198.185 77.16) (end 198.145 77.2) (width 0.707) (layer "B.Cu") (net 12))
 (segment (start 187.175 83.28) (end 187.175 84.03) (width 0.707) (layer "B.Cu") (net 12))
 (segment (start 187.175 78.72) (end 187.175 83.28) (width 0.707) (layer "B.Cu") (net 12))
 (segment (start 198.145 81.97) (end 196.085 84.03) (width 0.707) (layer "B.Cu") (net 12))
 (segment (start 187.335 83.28) (end 188.085 84.03) (width 0.707) (layer "B.Cu") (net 12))
 (segment (start 187.175 88.57) (end 187.045 88.7) (width 0.707) (layer "B.Cu") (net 12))
 (segment (start 187.175 84.03) (end 187.175 85.03) (width 0.707) (layer "B.Cu") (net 12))
 (segment (start 187.175 85.03) (end 187.175 88.57) (width 0.707) (layer "B.Cu") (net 12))
 (segment (start 213.425 104.69) (end 212.085 106.03) (width 0.707) (layer "B.Cu") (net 3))
 (segment (start 212.085 106.03) (end 181.835 106.03) (width 0.707) (layer "B.Cu") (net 3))
 (segment (start 181.835 106.03) (end 180.585 104.78) (width 0.707) (layer "B.Cu") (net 3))
 (segment (start 180.585 104.78) (end 180.585 98.31) (width 0.707) (layer "B.Cu") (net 3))
 (segment (start 213.425 102.56) (end 213.425 104.69) (width 0.707) (layer "B.Cu") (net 3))
 (segment (start 203.115 71.15) (end 203.115 72) (width 0.707) (layer "B.Cu") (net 16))
 (segment (start 200.725 75.64) (end 200.725 77.16) (width 0.707) (layer "B.Cu") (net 16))
 (segment (start 203.115 73.25) (end 200.725 75.64) (width 0.707) (layer "B.Cu") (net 16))
 (segment (start 203.115 71.35) (end 203.115 73.25) (width 0.707) (layer "B.Cu") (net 16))
 (segment (start 200.665 77.1) (end 200.725 77.16) (width 0.707) (layer "B.Cu") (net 16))
 (segment (start 206.315 70.25) (end 206.315 73.4) (width 0.707) (layer "B.Cu") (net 15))
 (segment (start 203.965 74.7) (end 203.265 75.4) (width 0.707) (layer "B.Cu") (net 15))
 (segment (start 200.575 71.35) (end 200.575 69.74) (width 0.707) (layer "B.Cu") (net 15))
 (segment (start 206.315 73.4) (end 205.015 74.7) (width 0.707) (layer "B.Cu") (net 15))
 (segment (start 205.015 74.7) (end 203.965 74.7) (width 0.707) (layer "B.Cu") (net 15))
 (segment (start 205.065 69) (end 206.315 70.25) (width 0.707) (layer "B.Cu") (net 15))
 (segment (start 201.315 69) (end 205.065 69) (width 0.707) (layer "B.Cu") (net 15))
 (segment (start 200.575 69.74) (end 201.315 69) (width 0.707) (layer "B.Cu") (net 15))
 (segment (start 203.265 75.4) (end 203.265 77.16) (width 0.707) (layer "B.Cu") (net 15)))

